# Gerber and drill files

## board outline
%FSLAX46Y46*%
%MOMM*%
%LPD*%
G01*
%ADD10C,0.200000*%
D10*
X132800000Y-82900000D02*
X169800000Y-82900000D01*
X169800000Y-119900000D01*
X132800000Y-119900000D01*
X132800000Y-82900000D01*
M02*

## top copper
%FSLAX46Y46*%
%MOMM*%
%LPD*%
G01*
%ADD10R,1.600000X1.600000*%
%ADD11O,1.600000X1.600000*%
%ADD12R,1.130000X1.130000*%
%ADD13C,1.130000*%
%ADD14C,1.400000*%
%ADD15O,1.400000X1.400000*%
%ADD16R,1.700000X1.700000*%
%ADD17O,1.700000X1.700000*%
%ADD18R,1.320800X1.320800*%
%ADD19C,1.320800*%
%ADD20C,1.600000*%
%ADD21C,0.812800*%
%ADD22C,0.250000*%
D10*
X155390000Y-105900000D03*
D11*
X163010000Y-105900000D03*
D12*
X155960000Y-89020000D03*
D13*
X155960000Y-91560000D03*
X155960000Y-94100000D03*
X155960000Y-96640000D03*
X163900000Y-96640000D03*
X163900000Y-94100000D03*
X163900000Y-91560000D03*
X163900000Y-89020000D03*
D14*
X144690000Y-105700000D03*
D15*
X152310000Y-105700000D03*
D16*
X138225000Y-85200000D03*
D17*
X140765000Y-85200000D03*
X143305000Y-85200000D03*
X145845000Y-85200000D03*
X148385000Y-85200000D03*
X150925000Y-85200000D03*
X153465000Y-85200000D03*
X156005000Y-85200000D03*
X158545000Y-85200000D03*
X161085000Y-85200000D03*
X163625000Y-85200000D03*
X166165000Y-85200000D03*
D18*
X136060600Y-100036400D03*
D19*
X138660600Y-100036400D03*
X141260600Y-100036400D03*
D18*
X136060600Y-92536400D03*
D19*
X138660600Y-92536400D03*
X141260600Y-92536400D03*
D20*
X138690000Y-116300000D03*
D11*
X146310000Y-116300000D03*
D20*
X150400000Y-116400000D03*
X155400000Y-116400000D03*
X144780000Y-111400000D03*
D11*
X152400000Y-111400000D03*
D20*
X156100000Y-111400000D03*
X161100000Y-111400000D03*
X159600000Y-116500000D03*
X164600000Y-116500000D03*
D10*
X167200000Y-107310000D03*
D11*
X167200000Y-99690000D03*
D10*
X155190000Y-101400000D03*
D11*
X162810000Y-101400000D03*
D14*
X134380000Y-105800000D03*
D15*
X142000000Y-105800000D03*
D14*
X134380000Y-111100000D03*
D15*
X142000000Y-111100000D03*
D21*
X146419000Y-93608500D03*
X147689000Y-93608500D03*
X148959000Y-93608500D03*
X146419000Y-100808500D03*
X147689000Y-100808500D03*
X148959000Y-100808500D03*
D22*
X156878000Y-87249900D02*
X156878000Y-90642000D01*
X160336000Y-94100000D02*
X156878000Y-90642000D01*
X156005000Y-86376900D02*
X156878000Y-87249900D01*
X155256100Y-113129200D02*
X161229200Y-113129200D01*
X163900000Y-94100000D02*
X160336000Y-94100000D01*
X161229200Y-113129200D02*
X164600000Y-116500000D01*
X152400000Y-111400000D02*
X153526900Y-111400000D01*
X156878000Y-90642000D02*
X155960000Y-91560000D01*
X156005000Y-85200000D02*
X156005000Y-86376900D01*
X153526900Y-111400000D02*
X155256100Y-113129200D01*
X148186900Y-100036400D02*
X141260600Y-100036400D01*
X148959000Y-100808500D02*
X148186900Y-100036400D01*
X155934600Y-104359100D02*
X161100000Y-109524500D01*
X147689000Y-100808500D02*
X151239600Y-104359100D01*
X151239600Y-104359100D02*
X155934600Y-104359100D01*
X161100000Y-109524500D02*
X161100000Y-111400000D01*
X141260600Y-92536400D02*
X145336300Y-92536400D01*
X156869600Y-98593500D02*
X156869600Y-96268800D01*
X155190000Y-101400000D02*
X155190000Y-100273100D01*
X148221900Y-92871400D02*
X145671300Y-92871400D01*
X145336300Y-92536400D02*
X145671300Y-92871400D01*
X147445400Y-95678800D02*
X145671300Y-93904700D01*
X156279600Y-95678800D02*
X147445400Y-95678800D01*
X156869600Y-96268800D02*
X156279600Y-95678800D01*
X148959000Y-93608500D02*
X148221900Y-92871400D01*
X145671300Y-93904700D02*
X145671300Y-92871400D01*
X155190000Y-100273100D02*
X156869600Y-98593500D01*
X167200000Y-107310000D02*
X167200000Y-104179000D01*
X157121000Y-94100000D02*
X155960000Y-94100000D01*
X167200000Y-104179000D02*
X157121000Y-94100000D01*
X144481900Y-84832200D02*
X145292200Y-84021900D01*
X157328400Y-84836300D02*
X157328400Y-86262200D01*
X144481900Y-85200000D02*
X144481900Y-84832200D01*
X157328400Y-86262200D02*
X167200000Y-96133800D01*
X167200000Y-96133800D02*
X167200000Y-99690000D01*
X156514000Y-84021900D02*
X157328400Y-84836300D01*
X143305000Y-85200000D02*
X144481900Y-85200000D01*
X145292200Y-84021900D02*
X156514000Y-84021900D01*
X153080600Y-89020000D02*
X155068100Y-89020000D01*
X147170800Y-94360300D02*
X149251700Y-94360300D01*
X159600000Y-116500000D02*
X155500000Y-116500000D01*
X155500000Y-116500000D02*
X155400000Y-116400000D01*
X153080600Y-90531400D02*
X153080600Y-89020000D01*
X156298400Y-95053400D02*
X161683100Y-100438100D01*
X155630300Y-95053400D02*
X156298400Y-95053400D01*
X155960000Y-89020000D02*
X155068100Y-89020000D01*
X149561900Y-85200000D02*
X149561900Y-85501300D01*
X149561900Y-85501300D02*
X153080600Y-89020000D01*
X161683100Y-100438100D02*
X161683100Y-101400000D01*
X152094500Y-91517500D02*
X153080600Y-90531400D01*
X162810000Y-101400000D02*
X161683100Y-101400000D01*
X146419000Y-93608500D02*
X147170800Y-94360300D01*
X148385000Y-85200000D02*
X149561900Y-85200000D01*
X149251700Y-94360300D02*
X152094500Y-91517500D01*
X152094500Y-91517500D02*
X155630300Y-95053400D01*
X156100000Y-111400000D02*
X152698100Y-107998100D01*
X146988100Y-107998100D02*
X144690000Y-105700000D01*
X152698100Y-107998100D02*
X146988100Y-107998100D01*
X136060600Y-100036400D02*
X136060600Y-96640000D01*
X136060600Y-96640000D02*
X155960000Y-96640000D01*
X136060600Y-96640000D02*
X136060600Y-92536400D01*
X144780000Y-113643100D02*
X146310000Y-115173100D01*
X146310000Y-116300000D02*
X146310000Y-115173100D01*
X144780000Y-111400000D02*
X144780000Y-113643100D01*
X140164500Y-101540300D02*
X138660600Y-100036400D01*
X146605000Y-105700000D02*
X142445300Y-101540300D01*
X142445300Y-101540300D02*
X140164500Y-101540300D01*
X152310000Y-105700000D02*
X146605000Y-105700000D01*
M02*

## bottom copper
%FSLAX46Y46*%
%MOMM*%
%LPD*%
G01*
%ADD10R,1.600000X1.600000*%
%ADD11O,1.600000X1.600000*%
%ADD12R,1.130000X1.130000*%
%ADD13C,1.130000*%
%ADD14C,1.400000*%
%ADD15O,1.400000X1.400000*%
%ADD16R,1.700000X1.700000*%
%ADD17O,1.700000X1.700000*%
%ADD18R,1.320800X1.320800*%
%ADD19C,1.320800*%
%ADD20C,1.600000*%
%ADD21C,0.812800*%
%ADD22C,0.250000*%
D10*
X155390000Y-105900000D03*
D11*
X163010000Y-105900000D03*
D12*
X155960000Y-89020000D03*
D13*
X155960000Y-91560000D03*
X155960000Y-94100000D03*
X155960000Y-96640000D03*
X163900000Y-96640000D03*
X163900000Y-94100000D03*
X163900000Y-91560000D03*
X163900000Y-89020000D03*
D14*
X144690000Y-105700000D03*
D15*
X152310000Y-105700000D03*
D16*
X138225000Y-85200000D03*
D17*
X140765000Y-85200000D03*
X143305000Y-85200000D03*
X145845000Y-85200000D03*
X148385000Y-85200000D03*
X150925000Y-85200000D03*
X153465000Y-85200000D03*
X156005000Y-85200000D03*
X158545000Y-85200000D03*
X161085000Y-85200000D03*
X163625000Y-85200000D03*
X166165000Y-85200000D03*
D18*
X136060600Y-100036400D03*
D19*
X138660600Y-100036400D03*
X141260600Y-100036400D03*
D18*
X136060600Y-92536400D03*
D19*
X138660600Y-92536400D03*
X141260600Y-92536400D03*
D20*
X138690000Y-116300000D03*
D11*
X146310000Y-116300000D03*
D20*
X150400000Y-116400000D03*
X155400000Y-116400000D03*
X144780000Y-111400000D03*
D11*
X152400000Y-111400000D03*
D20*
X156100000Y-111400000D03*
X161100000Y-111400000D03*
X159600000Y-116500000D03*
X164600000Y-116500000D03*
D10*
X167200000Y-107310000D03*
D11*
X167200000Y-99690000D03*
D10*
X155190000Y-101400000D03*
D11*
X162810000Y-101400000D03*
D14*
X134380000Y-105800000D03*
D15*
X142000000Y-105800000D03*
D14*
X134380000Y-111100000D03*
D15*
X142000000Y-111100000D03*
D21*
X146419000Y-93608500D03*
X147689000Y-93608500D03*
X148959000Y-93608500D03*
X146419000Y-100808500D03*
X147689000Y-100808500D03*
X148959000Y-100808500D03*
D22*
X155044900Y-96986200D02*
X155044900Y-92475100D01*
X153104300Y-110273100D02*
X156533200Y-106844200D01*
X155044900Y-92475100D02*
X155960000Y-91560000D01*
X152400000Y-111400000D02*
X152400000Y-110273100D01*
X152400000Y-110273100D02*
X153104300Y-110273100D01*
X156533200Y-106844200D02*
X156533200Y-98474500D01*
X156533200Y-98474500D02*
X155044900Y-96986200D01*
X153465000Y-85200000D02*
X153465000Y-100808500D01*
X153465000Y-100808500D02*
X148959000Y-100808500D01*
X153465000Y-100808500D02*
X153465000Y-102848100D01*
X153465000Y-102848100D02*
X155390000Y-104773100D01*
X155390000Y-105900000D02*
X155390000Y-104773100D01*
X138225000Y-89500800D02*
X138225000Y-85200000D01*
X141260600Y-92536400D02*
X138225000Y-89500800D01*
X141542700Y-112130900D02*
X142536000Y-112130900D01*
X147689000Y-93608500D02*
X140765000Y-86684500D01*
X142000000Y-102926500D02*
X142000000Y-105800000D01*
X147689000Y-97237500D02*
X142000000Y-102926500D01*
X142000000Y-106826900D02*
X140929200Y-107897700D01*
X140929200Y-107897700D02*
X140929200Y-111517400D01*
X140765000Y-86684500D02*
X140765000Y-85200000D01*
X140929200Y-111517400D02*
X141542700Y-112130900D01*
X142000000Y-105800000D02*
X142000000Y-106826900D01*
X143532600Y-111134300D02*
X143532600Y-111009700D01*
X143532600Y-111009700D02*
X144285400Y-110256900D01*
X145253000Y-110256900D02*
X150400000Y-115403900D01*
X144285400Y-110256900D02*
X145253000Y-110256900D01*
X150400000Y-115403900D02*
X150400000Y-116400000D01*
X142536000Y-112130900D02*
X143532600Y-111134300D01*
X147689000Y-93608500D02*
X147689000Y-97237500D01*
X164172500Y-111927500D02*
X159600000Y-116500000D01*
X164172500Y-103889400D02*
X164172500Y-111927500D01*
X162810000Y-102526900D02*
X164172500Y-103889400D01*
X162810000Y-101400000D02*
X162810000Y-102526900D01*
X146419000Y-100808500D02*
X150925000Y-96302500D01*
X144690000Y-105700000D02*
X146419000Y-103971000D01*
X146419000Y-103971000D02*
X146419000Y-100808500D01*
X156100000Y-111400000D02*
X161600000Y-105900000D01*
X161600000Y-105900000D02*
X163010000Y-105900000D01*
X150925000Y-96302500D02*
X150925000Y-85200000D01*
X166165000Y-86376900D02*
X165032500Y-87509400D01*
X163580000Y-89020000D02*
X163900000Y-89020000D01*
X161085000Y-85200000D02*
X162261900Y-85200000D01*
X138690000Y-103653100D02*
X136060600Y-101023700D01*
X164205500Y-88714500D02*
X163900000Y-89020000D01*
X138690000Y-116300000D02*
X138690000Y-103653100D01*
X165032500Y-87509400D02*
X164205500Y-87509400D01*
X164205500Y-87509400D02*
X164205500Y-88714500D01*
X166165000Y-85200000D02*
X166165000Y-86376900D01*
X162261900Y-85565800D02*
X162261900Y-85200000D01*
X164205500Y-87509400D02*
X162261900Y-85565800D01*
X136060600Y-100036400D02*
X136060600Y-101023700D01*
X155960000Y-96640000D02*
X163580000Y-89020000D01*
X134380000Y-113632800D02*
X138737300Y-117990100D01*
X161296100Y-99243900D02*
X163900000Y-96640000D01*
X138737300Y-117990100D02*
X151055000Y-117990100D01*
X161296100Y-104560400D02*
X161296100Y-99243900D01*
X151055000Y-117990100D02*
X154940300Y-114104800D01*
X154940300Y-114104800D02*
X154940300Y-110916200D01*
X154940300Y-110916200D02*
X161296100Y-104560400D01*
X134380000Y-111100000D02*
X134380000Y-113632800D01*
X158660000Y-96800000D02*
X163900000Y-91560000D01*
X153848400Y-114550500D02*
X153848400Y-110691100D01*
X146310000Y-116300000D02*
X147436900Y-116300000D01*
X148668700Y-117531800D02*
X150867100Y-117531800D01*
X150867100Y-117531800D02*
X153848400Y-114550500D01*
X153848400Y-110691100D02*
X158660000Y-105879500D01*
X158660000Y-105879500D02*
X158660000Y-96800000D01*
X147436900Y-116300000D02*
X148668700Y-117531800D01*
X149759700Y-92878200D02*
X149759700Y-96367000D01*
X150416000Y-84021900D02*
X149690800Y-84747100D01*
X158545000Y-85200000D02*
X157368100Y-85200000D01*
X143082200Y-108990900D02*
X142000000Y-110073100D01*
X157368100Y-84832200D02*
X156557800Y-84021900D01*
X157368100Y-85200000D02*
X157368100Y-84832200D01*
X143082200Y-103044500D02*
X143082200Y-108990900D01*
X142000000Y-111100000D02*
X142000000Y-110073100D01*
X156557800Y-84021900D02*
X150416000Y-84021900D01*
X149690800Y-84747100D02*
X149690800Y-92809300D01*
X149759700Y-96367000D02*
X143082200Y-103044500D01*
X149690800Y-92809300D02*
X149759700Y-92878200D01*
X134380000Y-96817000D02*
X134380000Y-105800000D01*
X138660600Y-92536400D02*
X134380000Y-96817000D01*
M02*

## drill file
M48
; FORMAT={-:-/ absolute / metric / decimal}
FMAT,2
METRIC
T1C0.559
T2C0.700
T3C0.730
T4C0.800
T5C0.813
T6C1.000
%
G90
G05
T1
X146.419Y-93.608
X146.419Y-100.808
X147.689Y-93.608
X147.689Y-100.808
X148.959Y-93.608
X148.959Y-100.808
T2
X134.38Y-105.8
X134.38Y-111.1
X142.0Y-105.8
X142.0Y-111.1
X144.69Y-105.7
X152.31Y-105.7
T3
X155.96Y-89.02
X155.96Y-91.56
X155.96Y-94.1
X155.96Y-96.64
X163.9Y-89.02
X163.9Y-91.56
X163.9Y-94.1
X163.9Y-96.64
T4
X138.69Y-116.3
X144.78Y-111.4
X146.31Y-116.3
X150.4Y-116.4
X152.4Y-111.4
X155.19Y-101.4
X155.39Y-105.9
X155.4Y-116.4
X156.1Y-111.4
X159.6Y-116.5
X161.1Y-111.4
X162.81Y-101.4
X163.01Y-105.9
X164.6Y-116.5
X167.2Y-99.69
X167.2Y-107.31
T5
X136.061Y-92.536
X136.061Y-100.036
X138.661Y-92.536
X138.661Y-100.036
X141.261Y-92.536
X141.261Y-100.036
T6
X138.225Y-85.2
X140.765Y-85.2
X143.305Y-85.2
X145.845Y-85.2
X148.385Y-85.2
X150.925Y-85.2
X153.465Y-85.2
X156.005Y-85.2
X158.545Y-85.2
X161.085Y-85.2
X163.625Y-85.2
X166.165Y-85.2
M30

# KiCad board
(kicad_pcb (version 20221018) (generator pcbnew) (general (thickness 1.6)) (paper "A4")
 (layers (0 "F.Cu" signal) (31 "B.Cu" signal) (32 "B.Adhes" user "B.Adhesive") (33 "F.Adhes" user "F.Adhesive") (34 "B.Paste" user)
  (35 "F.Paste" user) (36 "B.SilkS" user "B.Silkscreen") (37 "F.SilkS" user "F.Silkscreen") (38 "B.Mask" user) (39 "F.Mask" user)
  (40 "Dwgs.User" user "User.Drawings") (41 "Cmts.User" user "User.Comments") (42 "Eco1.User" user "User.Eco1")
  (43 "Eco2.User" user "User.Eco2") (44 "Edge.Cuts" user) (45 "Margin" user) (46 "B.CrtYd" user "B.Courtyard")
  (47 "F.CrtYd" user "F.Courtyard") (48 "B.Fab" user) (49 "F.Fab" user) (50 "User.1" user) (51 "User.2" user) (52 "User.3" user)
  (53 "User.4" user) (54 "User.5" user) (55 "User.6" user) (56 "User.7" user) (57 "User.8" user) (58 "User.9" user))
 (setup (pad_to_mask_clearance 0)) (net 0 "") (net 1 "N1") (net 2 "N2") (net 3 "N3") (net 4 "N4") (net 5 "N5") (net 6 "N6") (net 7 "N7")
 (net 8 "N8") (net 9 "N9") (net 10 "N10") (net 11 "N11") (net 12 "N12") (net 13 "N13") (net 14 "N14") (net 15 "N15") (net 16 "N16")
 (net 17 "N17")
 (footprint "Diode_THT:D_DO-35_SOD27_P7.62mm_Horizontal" (layer "F.Cu") (at 155.39 105.9)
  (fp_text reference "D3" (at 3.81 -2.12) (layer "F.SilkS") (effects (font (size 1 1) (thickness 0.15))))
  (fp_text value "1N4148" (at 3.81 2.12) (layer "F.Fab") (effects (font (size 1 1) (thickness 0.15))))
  (pad "1" thru_hole rect (at 0 0) (size 1.6 1.6) (drill 0.8) (layers "*.Cu" "*.Mask") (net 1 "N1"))
  (pad "2" thru_hole oval (at 7.62 0) (size 1.6 1.6) (drill 0.8) (layers "*.Cu" "*.Mask") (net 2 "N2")))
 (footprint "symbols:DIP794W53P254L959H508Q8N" (layer "F.Cu") (at 159.93 92.83)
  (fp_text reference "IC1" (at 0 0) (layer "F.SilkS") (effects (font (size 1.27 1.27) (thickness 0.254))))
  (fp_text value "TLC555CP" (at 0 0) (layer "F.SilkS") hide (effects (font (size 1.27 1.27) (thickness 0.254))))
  (pad "1" thru_hole rect (at -3.97 -3.81) (size 1.13 1.13) (drill 0.73) (layers "*.Cu" "*.Mask") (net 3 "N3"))
  (pad "2" thru_hole circle (at -3.97 -1.27) (size 1.13 1.13) (drill 0.73) (layers "*.Cu" "*.Mask") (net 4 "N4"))
  (pad "3" thru_hole circle (at -3.97 1.27) (size 1.13 1.13) (drill 0.73) (layers "*.Cu" "*.Mask") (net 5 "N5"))
  (pad "4" thru_hole circle (at -3.97 3.81) (size 1.13 1.13) (drill 0.73) (layers "*.Cu" "*.Mask") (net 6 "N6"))
  (pad "5" thru_hole circle (at 3.97 3.81) (size 1.13 1.13) (drill 0.73) (layers "*.Cu" "*.Mask") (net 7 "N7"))
  (pad "6" thru_hole circle (at 3.97 1.27) (size 1.13 1.13) (drill 0.73) (layers "*.Cu" "*.Mask") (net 4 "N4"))
  (pad "7" thru_hole circle (at 3.97 -1.27) (size 1.13 1.13) (drill 0.73) (layers "*.Cu" "*.Mask") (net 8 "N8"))
  (pad "8" thru_hole circle (at 3.97 -3.81) (size 1.13 1.13) (drill 0.73) (layers "*.Cu" "*.Mask") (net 6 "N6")))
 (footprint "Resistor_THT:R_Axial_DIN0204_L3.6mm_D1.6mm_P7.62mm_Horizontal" (layer "F.Cu") (at 144.69 105.7)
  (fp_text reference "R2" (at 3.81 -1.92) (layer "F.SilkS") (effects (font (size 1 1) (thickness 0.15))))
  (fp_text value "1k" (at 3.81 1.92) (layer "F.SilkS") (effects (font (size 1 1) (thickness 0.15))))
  (pad "1" thru_hole circle (at 0 0) (size 1.4 1.4) (drill 0.7) (layers "*.Cu" "*.Mask") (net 2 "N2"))
  (pad "2" thru_hole oval (at 7.62 0) (size 1.4 1.4) (drill 0.7) (layers "*.Cu" "*.Mask") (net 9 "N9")))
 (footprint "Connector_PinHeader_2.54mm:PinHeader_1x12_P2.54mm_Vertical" (layer "F.Cu") (at 138.225 85.2 90)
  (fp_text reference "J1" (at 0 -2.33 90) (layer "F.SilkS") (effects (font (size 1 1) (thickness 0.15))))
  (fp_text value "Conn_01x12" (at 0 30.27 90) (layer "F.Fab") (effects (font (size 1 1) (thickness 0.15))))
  (pad "1" thru_hole rect (at 0 0 90) (size 1.7 1.7) (drill 1) (layers "*.Cu" "*.Mask") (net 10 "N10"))
  (pad "2" thru_hole oval (at 0 2.54 90) (size 1.7 1.7) (drill 1) (layers "*.Cu" "*.Mask") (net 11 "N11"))
  (pad "3" thru_hole oval (at 0 5.08 90) (size 1.7 1.7) (drill 1) (layers "*.Cu" "*.Mask") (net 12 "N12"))
  (pad "4" thru_hole oval (at 0 7.62 90) (size 1.7 1.7) (drill 1) (layers "*.Cu" "*.Mask") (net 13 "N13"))
  (pad "5" thru_hole oval (at 0 10.16 90) (size 1.7 1.7) (drill 1) (layers "*.Cu" "*.Mask") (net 3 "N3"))
  (pad "6" thru_hole oval (at 0 12.7 90) (size 1.7 1.7) (drill 1) (layers "*.Cu" "*.Mask") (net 2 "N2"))
  (pad "7" thru_hole oval (at 0 15.24 90) (size 1.7 1.7) (drill 1) (layers "*.Cu" "*.Mask") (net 1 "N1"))
  (pad "8" thru_hole oval (at 0 17.78 90) (size 1.7 1.7) (drill 1) (layers "*.Cu" "*.Mask") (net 4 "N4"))
  (pad "9" thru_hole oval (at 0 20.32 90) (size 1.7 1.7) (drill 1) (layers "*.Cu" "*.Mask") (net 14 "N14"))
  (pad "10" thru_hole oval (at 0 22.86 90) (size 1.7 1.7) (drill 1) (layers "*.Cu" "*.Mask") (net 6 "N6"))
  (pad "11" thru_hole oval (at 0 25.4 90) (size 1.7 1.7) (drill 1) (layers "*.Cu" "*.Mask") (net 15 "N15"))
  (pad "12" thru_hole oval (at 0 27.94 90) (size 1.7 1.7) (drill 1) (layers "*.Cu" "*.Mask") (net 6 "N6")))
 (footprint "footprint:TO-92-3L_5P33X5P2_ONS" (layer "F.Cu") (at 136.0606 100.0364)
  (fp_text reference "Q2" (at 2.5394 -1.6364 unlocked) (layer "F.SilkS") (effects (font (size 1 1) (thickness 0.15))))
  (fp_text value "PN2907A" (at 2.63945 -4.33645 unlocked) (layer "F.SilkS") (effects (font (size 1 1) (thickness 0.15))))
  (pad "1" thru_hole rect (at 0 0) (size 1.3208 1.3208) (drill 0.8128) (layers "*.Cu" "*.Mask") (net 6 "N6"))
  (pad "2" thru_hole circle (at 2.6 0) (size 1.3208 1.3208) (drill 0.8128) (layers "*.Cu" "*.Mask") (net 9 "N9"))
  (pad "3" thru_hole circle (at 5.2 0) (size 1.3208 1.3208) (drill 0.8128) (layers "*.Cu" "*.Mask") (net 1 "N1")))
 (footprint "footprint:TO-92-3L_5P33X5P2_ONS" (layer "F.Cu") (at 136.0606 92.5364)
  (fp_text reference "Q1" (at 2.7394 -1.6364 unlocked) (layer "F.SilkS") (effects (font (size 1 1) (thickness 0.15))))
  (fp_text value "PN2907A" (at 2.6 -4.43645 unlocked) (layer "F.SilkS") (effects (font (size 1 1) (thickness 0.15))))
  (pad "1" thru_hole rect (at 0 0) (size 1.3208 1.3208) (drill 0.8128) (layers "*.Cu" "*.Mask") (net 6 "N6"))
  (pad "2" thru_hole circle (at 2.6 0) (size 1.3208 1.3208) (drill 0.8128) (layers "*.Cu" "*.Mask") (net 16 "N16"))
  (pad "3" thru_hole circle (at 5.2 0) (size 1.3208 1.3208) (drill 0.8128) (layers "*.Cu" "*.Mask") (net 10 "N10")))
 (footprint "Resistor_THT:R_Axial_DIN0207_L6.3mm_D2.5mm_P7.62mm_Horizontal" (layer "F.Cu") (at 138.69 116.3)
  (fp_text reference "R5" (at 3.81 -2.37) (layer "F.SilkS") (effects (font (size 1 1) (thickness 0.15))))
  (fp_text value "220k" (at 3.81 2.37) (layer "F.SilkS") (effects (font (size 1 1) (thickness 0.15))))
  (pad "1" thru_hole circle (at 0 0) (size 1.6 1.6) (drill 0.8) (layers "*.Cu" "*.Mask") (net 6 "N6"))
  (pad "2" thru_hole oval (at 7.62 0) (size 1.6 1.6) (drill 0.8) (layers "*.Cu" "*.Mask") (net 8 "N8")))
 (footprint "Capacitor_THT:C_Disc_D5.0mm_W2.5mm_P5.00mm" (layer "F.Cu") (at 150.4 116.4)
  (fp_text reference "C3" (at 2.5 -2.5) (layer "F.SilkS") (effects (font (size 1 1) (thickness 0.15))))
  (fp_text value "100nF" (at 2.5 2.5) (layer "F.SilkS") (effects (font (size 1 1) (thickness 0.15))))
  (pad "1" thru_hole circle (at 0 0) (size 1.6 1.6) (drill 0.8) (layers "*.Cu" "*.Mask") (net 11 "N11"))
  (pad "2" thru_hole circle (at 5 0) (size 1.6 1.6) (drill 0.8) (layers "*.Cu" "*.Mask") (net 3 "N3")))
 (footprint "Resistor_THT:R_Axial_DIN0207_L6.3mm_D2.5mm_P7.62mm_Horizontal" (layer "F.Cu") (at 144.78 111.4)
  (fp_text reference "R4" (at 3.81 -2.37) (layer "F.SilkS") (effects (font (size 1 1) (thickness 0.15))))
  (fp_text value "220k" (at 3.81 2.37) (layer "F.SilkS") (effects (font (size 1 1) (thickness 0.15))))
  (pad "1" thru_hole circle (at 0 0) (size 1.6 1.6) (drill 0.8) (layers "*.Cu" "*.Mask") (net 8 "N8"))
  (pad "2" thru_hole oval (at 7.62 0) (size 1.6 1.6) (drill 0.8) (layers "*.Cu" "*.Mask") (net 4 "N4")))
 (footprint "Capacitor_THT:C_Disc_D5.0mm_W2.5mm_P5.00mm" (layer "F.Cu") (at 156.1 111.4)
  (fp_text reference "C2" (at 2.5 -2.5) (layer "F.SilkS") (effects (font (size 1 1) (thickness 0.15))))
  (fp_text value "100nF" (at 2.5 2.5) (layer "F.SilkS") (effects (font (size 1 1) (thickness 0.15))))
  (pad "1" thru_hole circle (at 0 0) (size 1.6 1.6) (drill 0.8) (layers "*.Cu" "*.Mask") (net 2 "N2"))
  (pad "2" thru_hole circle (at 5 0) (size 1.6 1.6) (drill 0.8) (layers "*.Cu" "*.Mask") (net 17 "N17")))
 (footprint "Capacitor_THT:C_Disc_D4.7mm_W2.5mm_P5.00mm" (layer "F.Cu") (at 159.6 116.5)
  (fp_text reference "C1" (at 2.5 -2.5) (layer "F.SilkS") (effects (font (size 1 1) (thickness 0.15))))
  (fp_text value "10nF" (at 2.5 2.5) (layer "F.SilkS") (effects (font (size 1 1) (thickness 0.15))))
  (pad "1" thru_hole circle (at 0 0) (size 1.6 1.6) (drill 0.8) (layers "*.Cu" "*.Mask") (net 3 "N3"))
  (pad "2" thru_hole circle (at 5 0) (size 1.6 1.6) (drill 0.8) (layers "*.Cu" "*.Mask") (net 4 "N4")))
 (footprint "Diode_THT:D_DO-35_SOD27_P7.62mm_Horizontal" (layer "F.Cu") (at 167.2 107.31 90)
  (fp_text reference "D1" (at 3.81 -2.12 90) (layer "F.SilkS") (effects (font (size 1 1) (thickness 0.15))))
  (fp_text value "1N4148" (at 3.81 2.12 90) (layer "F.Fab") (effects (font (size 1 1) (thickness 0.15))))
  (pad "1" thru_hole rect (at 0 0 90) (size 1.6 1.6) (drill 0.8) (layers "*.Cu" "*.Mask") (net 5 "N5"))
  (pad "2" thru_hole oval (at 7.62 0 90) (size 1.6 1.6) (drill 0.8) (layers "*.Cu" "*.Mask") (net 12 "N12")))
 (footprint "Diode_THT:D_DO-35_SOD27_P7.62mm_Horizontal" (layer "F.Cu") (at 155.19 101.4)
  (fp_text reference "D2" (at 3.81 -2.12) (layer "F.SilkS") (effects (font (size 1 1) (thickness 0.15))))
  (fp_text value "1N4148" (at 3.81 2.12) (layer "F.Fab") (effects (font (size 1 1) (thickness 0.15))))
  (pad "1" thru_hole rect (at 0 0) (size 1.6 1.6) (drill 0.8) (layers "*.Cu" "*.Mask") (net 10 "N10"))
  (pad "2" thru_hole oval (at 7.62 0) (size 1.6 1.6) (drill 0.8) (layers "*.Cu" "*.Mask") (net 3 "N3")))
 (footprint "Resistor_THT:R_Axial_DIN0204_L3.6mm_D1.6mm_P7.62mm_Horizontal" (layer "F.Cu") (at 134.38 105.8)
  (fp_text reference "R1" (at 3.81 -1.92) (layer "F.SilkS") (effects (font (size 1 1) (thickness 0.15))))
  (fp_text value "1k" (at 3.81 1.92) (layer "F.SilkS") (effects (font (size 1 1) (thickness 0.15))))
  (pad "1" thru_hole circle (at 0 0) (size 1.4 1.4) (drill 0.7) (layers "*.Cu" "*.Mask") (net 16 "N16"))
  (pad "2" thru_hole oval (at 7.62 0) (size 1.4 1.4) (drill 0.7) (layers "*.Cu" "*.Mask") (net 11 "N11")))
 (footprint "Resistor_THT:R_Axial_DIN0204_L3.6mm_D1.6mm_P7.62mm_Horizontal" (layer "F.Cu") (at 134.38 111.1)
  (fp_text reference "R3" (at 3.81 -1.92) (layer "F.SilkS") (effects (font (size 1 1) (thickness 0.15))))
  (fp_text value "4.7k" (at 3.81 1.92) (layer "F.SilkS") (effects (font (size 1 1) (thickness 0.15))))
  (pad "1" thru_hole circle (at 0 0) (size 1.4 1.4) (drill 0.7) (layers "*.Cu" "*.Mask") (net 7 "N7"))
  (pad "2" thru_hole oval (at 7.62 0) (size 1.4 1.4) (drill 0.7) (layers "*.Cu" "*.Mask") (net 14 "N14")))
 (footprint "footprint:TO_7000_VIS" (layer "F.Cu") (at 146.419 93.6085)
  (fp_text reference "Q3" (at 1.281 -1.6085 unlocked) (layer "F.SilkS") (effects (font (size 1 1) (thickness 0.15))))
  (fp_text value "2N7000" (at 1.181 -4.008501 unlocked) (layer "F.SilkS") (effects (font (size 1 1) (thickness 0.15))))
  (pad "1" thru_hole circle (at 0 0) (size 0.8128 0.8128) (drill 0.5588) (layers "*.Cu" "*.Mask") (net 3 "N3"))
  (pad "2" thru_hole circle (at 1.27 0) (size 0.8128 0.8128) (drill 0.5588) (layers "*.Cu" "*.Mask") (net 11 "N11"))
  (pad "3" thru_hole circle (at 2.54 0) (size 0.8128 0.8128) (drill 0.5588) (layers "*.Cu" "*.Mask") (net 10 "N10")))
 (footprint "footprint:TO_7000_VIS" (layer "F.Cu") (at 146.419 100.8085)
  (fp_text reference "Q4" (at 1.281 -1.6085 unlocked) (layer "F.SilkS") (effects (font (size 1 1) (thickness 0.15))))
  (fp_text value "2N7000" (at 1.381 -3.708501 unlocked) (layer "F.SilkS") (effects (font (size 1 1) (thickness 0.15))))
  (pad "1" thru_hole circle (at 0 0) (size 0.8128 0.8128) (drill 0.5588) (layers "*.Cu" "*.Mask") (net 2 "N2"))
  (pad "2" thru_hole circle (at 1.27 0) (size 0.8128 0.8128) (drill 0.5588) (layers "*.Cu" "*.Mask") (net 17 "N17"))
  (pad "3" thru_hole circle (at 2.54 0) (size 0.8128 0.8128) (drill 0.5588) (layers "*.Cu" "*.Mask") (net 1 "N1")))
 (gr_rect (start 132.8 82.9) (end 169.8 119.9) (stroke (width 0.2) (type default)) (fill none) (layer "Edge.Cuts"))
 (segment (start 156.878 87.2499) (end 156.878 90.642) (width 0.25) (layer "F.Cu") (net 4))
 (segment (start 160.336 94.1) (end 156.878 90.642) (width 0.25) (layer "F.Cu") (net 4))
 (segment (start 156.005 86.3769) (end 156.878 87.2499) (width 0.25) (layer "F.Cu") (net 4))
 (segment (start 155.2561 113.1292) (end 161.2292 113.1292) (width 0.25) (layer "F.Cu") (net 4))
 (segment (start 163.9 94.1) (end 160.336 94.1) (width 0.25) (layer "F.Cu") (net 4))
 (segment (start 161.2292 113.1292) (end 164.6 116.5) (width 0.25) (layer "F.Cu") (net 4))
 (segment (start 152.4 111.4) (end 153.5269 111.4) (width 0.25) (layer "F.Cu") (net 4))
 (segment (start 156.878 90.642) (end 155.96 91.56) (width 0.25) (layer "F.Cu") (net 4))
 (segment (start 156.005 85.2) (end 156.005 86.3769) (width 0.25) (layer "F.Cu") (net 4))
 (segment (start 153.5269 111.4) (end 155.2561 113.1292) (width 0.25) (layer "F.Cu") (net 4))
 (segment (start 155.0449 96.9862) (end 155.0449 92.4751) (width 0.25) (layer "B.Cu") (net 4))
 (segment (start 153.1043 110.2731) (end 156.5332 106.8442) (width 0.25) (layer "B.Cu") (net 4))
 (segment (start 155.0449 92.4751) (end 155.96 91.56) (width 0.25) (layer "B.Cu") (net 4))
 (segment (start 152.4 111.4) (end 152.4 110.2731) (width 0.25) (layer "B.Cu") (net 4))
 (segment (start 152.4 110.2731) (end 153.1043 110.2731) (width 0.25) (layer "B.Cu") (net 4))
 (segment (start 156.5332 106.8442) (end 156.5332 98.4745) (width 0.25) (layer "B.Cu") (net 4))
 (segment (start 156.5332 98.4745) (end 155.0449 96.9862) (width 0.25) (layer "B.Cu") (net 4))
 (segment (start 148.1869 100.0364) (end 141.2606 100.0364) (width 0.25) (layer "F.Cu") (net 1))
 (segment (start 148.959 100.8085) (end 148.1869 100.0364) (width 0.25) (layer "F.Cu") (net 1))
 (segment (start 153.465 85.2) (end 153.465 100.8085) (width 0.25) (layer "B.Cu") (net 1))
 (segment (start 153.465 100.8085) (end 148.959 100.8085) (width 0.25) (layer "B.Cu") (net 1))
 (segment (start 153.465 100.8085) (end 153.465 102.8481) (width 0.25) (layer "B.Cu") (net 1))
 (segment (start 153.465 102.8481) (end 155.39 104.7731) (width 0.25) (layer "B.Cu") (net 1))
 (segment (start 155.39 105.9) (end 155.39 104.7731) (width 0.25) (layer "B.Cu") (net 1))
 (segment (start 155.9346 104.3591) (end 161.1 109.5245) (width 0.25) (layer "F.Cu") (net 17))
 (segment (start 147.689 100.8085) (end 151.2396 104.3591) (width 0.25) (layer "F.Cu") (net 17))
 (segment (start 151.2396 104.3591) (end 155.9346 104.3591) (width 0.25) (layer "F.Cu") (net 17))
 (segment (start 161.1 109.5245) (end 161.1 111.4) (width 0.25) (layer "F.Cu") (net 17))
 (segment (start 141.2606 92.5364) (end 145.3363 92.5364) (width 0.25) (layer "F.Cu") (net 10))
 (segment (start 156.8696 98.5935) (end 156.8696 96.2688) (width 0.25) (layer "F.Cu") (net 10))
 (segment (start 155.19 101.4) (end 155.19 100.2731) (width 0.25) (layer "F.Cu") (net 10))
 (segment (start 148.2219 92.8714) (end 145.6713 92.8714) (width 0.25) (layer "F.Cu") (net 10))
 (segment (start 145.3363 92.5364) (end 145.6713 92.8714) (width 0.25) (layer "F.Cu") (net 10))
 (segment (start 147.4454 95.6788) (end 145.6713 93.9047) (width 0.25) (layer "F.Cu") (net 10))
 (segment (start 156.2796 95.6788) (end 147.4454 95.6788) (width 0.25) (layer "F.Cu") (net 10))
 (segment (start 156.8696 96.2688) (end 156.2796 95.6788) (width 0.25) (layer "F.Cu") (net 10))
 (segment (start 148.959 93.6085) (end 148.2219 92.8714) (width 0.25) (layer "F.Cu") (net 10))
 (segment (start 145.6713 93.9047) (end 145.6713 92.8714) (width 0.25) (layer "F.Cu") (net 10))
 (segment (start 155.19 100.2731) (end 156.8696 98.5935) (width 0.25) (layer "F.Cu") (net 10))
 (segment (start 138.225 89.5008) (end 138.225 85.2) (width 0.25) (layer "B.Cu") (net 10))
 (segment (start 141.2606 92.5364) (end 138.225 89.5008) (width 0.25) (layer "B.Cu") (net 10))
 (segment (start 141.5427 112.1309) (end 142.536 112.1309) (width 0.25) (layer "B.Cu") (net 11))
 (segment (start 147.689 93.6085) (end 140.765 86.6845) (width 0.25) (layer "B.Cu") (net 11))
 (segment (start 142 102.9265) (end 142 105.8) (width 0.25) (layer "B.Cu") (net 11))
 (segment (start 147.689 97.2375) (end 142 102.9265) (width 0.25) (layer "B.Cu") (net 11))
 (segment (start 142 106.8269) (end 140.9292 107.8977) (width 0.25) (layer "B.Cu") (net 11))
 (segment (start 140.9292 107.8977) (end 140.9292 111.5174) (width 0.25) (layer "B.Cu") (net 11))
 (segment (start 140.765 86.6845) (end 140.765 85.2) (width 0.25) (layer "B.Cu") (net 11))
 (segment (start 140.9292 111.5174) (end 141.5427 112.1309) (width 0.25) (layer "B.Cu") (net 11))
 (segment (start 142 105.8) (end 142 106.8269) (width 0.25) (layer "B.Cu") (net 11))
 (segment (start 143.5326 111.1343) (end 143.5326 111.0097) (width 0.25) (layer "B.Cu") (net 11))
 (segment (start 143.5326 111.0097) (end 144.2854 110.2569) (width 0.25) (layer "B.Cu") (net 11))
 (segment (start 145.253 110.2569) (end 150.4 115.4039) (width 0.25) (layer "B.Cu") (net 11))
 (segment (start 144.2854 110.2569) (end 145.253 110.2569) (width 0.25) (layer "B.Cu") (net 11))
 (segment (start 150.4 115.4039) (end 150.4 116.4) (width 0.25) (layer "B.Cu") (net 11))
 (segment (start 142.536 112.1309) (end 143.5326 111.1343) (width 0.25) (layer "B.Cu") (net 11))
 (segment (start 147.689 93.6085) (end 147.689 97.2375) (width 0.25) (layer "B.Cu") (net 11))
 (segment (start 167.2 107.31) (end 167.2 104.179) (width 0.25) (layer "F.Cu") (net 5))
 (segment (start 157.121 94.1) (end 155.96 94.1) (width 0.25) (layer "F.Cu") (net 5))
 (segment (start 167.2 104.179) (end 157.121 94.1) (width 0.25) (layer "F.Cu") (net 5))
 (segment (start 144.4819 84.8322) (end 145.2922 84.0219) (width 0.25) (layer "F.Cu") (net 12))
 (segment (start 157.3284 84.8363) (end 157.3284 86.2622) (width 0.25) (layer "F.Cu") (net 12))
 (segment (start 144.4819 85.2) (end 144.4819 84.8322) (width 0.25) (layer "F.Cu") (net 12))
 (segment (start 157.3284 86.2622) (end 167.2 96.1338) (width 0.25) (layer "F.Cu") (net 12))
 (segment (start 167.2 96.1338) (end 167.2 99.69) (width 0.25) (layer "F.Cu") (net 12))
 (segment (start 156.514 84.0219) (end 157.3284 84.8363) (width 0.25) (layer "F.Cu") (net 12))
 (segment (start 143.305 85.2) (end 144.4819 85.2) (width 0.25) (layer "F.Cu") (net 12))
 (segment (start 145.2922 84.0219) (end 156.514 84.0219) (width 0.25) (layer "F.Cu") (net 12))
 (segment (start 153.0806 89.02) (end 155.0681 89.02) (width 0.25) (layer "F.Cu") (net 3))
 (segment (start 147.1708 94.3603) (end 149.2517 94.3603) (width 0.25) (layer "F.Cu") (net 3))
 (segment (start 159.6 116.5) (end 155.5 116.5) (width 0.25) (layer "F.Cu") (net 3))
 (segment (start 155.5 116.5) (end 155.4 116.4) (width 0.25) (layer "F.Cu") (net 3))
 (segment (start 153.0806 90.5314) (end 153.0806 89.02) (width 0.25) (layer "F.Cu") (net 3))
 (segment (start 156.2984 95.0534) (end 161.6831 100.4381) (width 0.25) (layer "F.Cu") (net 3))
 (segment (start 155.6303 95.0534) (end 156.2984 95.0534) (width 0.25) (layer "F.Cu") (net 3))
 (segment (start 155.96 89.02) (end 155.0681 89.02) (width 0.25) (layer "F.Cu") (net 3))
 (segment (start 149.5619 85.2) (end 149.5619 85.5013) (width 0.25) (layer "F.Cu") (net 3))
 (segment (start 149.5619 85.5013) (end 153.0806 89.02) (width 0.25) (layer "F.Cu") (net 3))
 (segment (start 161.6831 100.4381) (end 161.6831 101.4) (width 0.25) (layer "F.Cu") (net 3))
 (segment (start 152.0945 91.5175) (end 153.0806 90.5314) (width 0.25) (layer "F.Cu") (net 3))
 (segment (start 162.81 101.4) (end 161.6831 101.4) (width 0.25) (layer "F.Cu") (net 3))
 (segment (start 146.419 93.6085) (end 147.1708 94.3603) (width 0.25) (layer "F.Cu") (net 3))
 (segment (start 148.385 85.2) (end 149.5619 85.2) (width 0.25) (layer "F.Cu") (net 3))
 (segment (start 149.2517 94.3603) (end 152.0945 91.5175) (width 0.25) (layer "F.Cu") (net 3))
 (segment (start 152.0945 91.5175) (end 155.6303 95.0534) (width 0.25) (layer "F.Cu") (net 3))
 (segment (start 164.1725 111.9275) (end 159.6 116.5) (width 0.25) (layer "B.Cu") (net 3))
 (segment (start 164.1725 103.8894) (end 164.1725 111.9275) (width 0.25) (layer "B.Cu") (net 3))
 (segment (start 162.81 102.5269) (end 164.1725 103.8894) (width 0.25) (layer "B.Cu") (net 3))
 (segment (start 162.81 101.4) (end 162.81 102.5269) (width 0.25) (layer "B.Cu") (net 3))
 (segment (start 156.1 111.4) (end 152.6981 107.9981) (width 0.25) (layer "F.Cu") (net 2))
 (segment (start 146.9881 107.9981) (end 144.69 105.7) (width 0.25) (layer "F.Cu") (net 2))
 (segment (start 152.6981 107.9981) (end 146.9881 107.9981) (width 0.25) (layer "F.Cu") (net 2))
 (segment (start 146.419 100.8085) (end 150.925 96.3025) (width 0.25) (layer "B.Cu") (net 2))
 (segment (start 144.69 105.7) (end 146.419 103.971) (width 0.25) (layer "B.Cu") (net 2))
 (segment (start 146.419 103.971) (end 146.419 100.8085) (width 0.25) (layer "B.Cu") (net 2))
 (segment (start 156.1 111.4) (end 161.6 105.9) (width 0.25) (layer "B.Cu") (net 2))
 (segment (start 161.6 105.9) (end 163.01 105.9) (width 0.25) (layer "B.Cu") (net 2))
 (segment (start 150.925 96.3025) (end 150.925 85.2) (width 0.25) (layer "B.Cu") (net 2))
 (segment (start 136.0606 100.0364) (end 136.0606 96.64) (width 0.25) (layer "F.Cu") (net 6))
 (segment (start 136.0606 96.64) (end 155.96 96.64) (width 0.25) (layer "F.Cu") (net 6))
 (segment (start 136.0606 96.64) (end 136.0606 92.5364) (width 0.25) (layer "F.Cu") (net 6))
 (segment (start 166.165 86.3769) (end 165.0325 87.5094) (width 0.25) (layer "B.Cu") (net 6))
 (segment (start 163.58 89.02) (end 163.9 89.02) (width 0.25) (layer "B.Cu") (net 6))
 (segment (start 161.085 85.2) (end 162.2619 85.2) (width 0.25) (layer "B.Cu") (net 6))
 (segment (start 138.69 103.6531) (end 136.0606 101.0237) (width 0.25) (layer "B.Cu") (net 6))
 (segment (start 164.2055 88.7145) (end 163.9 89.02) (width 0.25) (layer "B.Cu") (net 6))
 (segment (start 138.69 116.3) (end 138.69 103.6531) (width 0.25) (layer "B.Cu") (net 6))
 (segment (start 165.0325 87.5094) (end 164.2055 87.5094) (width 0.25) (layer "B.Cu") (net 6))
 (segment (start 164.2055 87.5094) (end 164.2055 88.7145) (width 0.25) (layer "B.Cu") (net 6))
 (segment (start 166.165 85.2) (end 166.165 86.3769) (width 0.25) (layer "B.Cu") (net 6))
 (segment (start 162.2619 85.5658) (end 162.2619 85.2) (width 0.25) (layer "B.Cu") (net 6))
 (segment (start 164.2055 87.5094) (end 162.2619 85.5658) (width 0.25) (layer "B.Cu") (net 6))
 (segment (start 136.0606 100.0364) (end 136.0606 101.0237) (width 0.25) (layer "B.Cu") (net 6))
 (segment (start 155.96 96.64) (end 163.58 89.02) (width 0.25) (layer "B.Cu") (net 6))
 (segment (start 134.38 113.6328) (end 138.7373 117.9901) (width 0.25) (layer "B.Cu") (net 7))
 (segment (start 161.2961 99.2439) (end 163.9 96.64) (width 0.25) (layer "B.Cu") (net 7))
 (segment (start 138.7373 117.9901) (end 151.055 117.9901) (width 0.25) (layer "B.Cu") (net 7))
 (segment (start 161.2961 104.5604) (end 161.2961 99.2439) (width 0.25) (layer "B.Cu") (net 7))
 (segment (start 151.055 117.9901) (end 154.9403 114.1048) (width 0.25) (layer "B.Cu") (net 7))
 (segment (start 154.9403 114.1048) (end 154.9403 110.9162) (width 0.25) (layer "B.Cu") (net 7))
 (segment (start 154.9403 110.9162) (end 161.2961 104.5604) (width 0.25) (layer "B.Cu") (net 7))
 (segment (start 134.38 111.1) (end 134.38 113.6328) (width 0.25) (layer "B.Cu") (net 7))
 (segment (start 144.78 113.6431) (end 146.31 115.1731) (width 0.25) (layer "F.Cu") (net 8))
 (segment (start 146.31 116.3) (end 146.31 115.1731) (width 0.25) (layer "F.Cu") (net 8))
 (segment (start 144.78 111.4) (end 144.78 113.6431) (width 0.25) (layer "F.Cu") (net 8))
 (segment (start 158.66 96.8) (end 163.9 91.56) (width 0.25) (layer "B.Cu") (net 8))
 (segment (start 153.8484 114.5505) (end 153.8484 110.6911) (width 0.25) (layer "B.Cu") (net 8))
 (segment (start 146.31 116.3) (end 147.4369 116.3) (width 0.25) (layer "B.Cu") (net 8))
 (segment (start 148.6687 117.5318) (end 150.8671 117.5318) (width 0.25) (layer "B.Cu") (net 8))
 (segment (start 150.8671 117.5318) (end 153.8484 114.5505) (width 0.25) (layer "B.Cu") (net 8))
 (segment (start 153.8484 110.6911) (end 158.66 105.8795) (width 0.25) (layer "B.Cu") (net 8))
 (segment (start 158.66 105.8795) (end 158.66 96.8) (width 0.25) (layer "B.Cu") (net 8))
 (segment (start 147.4369 116.3) (end 148.6687 117.5318) (width 0.25) (layer "B.Cu") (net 8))
 (segment (start 149.7597 92.8782) (end 149.7597 96.367) (width 0.25) (layer "B.Cu") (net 14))
 (segment (start 150.416 84.0219) (end 149.6908 84.7471) (width 0.25) (layer "B.Cu") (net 14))
 (segment (start 158.545 85.2) (end 157.3681 85.2) (width 0.25) (layer "B.Cu") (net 14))
 (segment (start 143.0822 108.9909) (end 142 110.0731) (width 0.25) (layer "B.Cu") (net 14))
 (segment (start 157.3681 84.8322) (end 156.5578 84.0219) (width 0.25) (layer "B.Cu") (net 14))
 (segment (start 157.3681 85.2) (end 157.3681 84.8322) (width 0.25) (layer "B.Cu") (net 14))
 (segment (start 143.0822 103.0445) (end 143.0822 108.9909) (width 0.25) (layer "B.Cu") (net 14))
 (segment (start 142 111.1) (end 142 110.0731) (width 0.25) (layer "B.Cu") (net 14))
 (segment (start 156.5578 84.0219) (end 150.416 84.0219) (width 0.25) (layer "B.Cu") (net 14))
 (segment (start 149.6908 84.7471) (end 149.6908 92.8093) (width 0.25) (layer "B.Cu") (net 14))
 (segment (start 149.7597 96.367) (end 143.0822 103.0445) (width 0.25) (layer "B.Cu") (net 14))
 (segment (start 149.6908 92.8093) (end 149.7597 92.8782) (width 0.25) (layer "B.Cu") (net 14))
 (segment (start 134.38 96.817) (end 134.38 105.8) (width 0.25) (layer "B.Cu") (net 16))
 (segment (start 138.6606 92.5364) (end 134.38 96.817) (width 0.25) (layer "B.Cu") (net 16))
 (segment (start 140.1645 101.5403) (end 138.6606 100.0364) (width 0.25) (layer "F.Cu") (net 9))
 (segment (start 146.605 105.7) (end 142.4453 101.5403) (width 0.25) (layer "F.Cu") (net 9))
 (segment (start 142.4453 101.5403) (end 140.1645 101.5403) (width 0.25) (layer "F.Cu") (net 9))
 (segment (start 152.31 105.7) (end 146.605 105.7) (width 0.25) (layer "F.Cu") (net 9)))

